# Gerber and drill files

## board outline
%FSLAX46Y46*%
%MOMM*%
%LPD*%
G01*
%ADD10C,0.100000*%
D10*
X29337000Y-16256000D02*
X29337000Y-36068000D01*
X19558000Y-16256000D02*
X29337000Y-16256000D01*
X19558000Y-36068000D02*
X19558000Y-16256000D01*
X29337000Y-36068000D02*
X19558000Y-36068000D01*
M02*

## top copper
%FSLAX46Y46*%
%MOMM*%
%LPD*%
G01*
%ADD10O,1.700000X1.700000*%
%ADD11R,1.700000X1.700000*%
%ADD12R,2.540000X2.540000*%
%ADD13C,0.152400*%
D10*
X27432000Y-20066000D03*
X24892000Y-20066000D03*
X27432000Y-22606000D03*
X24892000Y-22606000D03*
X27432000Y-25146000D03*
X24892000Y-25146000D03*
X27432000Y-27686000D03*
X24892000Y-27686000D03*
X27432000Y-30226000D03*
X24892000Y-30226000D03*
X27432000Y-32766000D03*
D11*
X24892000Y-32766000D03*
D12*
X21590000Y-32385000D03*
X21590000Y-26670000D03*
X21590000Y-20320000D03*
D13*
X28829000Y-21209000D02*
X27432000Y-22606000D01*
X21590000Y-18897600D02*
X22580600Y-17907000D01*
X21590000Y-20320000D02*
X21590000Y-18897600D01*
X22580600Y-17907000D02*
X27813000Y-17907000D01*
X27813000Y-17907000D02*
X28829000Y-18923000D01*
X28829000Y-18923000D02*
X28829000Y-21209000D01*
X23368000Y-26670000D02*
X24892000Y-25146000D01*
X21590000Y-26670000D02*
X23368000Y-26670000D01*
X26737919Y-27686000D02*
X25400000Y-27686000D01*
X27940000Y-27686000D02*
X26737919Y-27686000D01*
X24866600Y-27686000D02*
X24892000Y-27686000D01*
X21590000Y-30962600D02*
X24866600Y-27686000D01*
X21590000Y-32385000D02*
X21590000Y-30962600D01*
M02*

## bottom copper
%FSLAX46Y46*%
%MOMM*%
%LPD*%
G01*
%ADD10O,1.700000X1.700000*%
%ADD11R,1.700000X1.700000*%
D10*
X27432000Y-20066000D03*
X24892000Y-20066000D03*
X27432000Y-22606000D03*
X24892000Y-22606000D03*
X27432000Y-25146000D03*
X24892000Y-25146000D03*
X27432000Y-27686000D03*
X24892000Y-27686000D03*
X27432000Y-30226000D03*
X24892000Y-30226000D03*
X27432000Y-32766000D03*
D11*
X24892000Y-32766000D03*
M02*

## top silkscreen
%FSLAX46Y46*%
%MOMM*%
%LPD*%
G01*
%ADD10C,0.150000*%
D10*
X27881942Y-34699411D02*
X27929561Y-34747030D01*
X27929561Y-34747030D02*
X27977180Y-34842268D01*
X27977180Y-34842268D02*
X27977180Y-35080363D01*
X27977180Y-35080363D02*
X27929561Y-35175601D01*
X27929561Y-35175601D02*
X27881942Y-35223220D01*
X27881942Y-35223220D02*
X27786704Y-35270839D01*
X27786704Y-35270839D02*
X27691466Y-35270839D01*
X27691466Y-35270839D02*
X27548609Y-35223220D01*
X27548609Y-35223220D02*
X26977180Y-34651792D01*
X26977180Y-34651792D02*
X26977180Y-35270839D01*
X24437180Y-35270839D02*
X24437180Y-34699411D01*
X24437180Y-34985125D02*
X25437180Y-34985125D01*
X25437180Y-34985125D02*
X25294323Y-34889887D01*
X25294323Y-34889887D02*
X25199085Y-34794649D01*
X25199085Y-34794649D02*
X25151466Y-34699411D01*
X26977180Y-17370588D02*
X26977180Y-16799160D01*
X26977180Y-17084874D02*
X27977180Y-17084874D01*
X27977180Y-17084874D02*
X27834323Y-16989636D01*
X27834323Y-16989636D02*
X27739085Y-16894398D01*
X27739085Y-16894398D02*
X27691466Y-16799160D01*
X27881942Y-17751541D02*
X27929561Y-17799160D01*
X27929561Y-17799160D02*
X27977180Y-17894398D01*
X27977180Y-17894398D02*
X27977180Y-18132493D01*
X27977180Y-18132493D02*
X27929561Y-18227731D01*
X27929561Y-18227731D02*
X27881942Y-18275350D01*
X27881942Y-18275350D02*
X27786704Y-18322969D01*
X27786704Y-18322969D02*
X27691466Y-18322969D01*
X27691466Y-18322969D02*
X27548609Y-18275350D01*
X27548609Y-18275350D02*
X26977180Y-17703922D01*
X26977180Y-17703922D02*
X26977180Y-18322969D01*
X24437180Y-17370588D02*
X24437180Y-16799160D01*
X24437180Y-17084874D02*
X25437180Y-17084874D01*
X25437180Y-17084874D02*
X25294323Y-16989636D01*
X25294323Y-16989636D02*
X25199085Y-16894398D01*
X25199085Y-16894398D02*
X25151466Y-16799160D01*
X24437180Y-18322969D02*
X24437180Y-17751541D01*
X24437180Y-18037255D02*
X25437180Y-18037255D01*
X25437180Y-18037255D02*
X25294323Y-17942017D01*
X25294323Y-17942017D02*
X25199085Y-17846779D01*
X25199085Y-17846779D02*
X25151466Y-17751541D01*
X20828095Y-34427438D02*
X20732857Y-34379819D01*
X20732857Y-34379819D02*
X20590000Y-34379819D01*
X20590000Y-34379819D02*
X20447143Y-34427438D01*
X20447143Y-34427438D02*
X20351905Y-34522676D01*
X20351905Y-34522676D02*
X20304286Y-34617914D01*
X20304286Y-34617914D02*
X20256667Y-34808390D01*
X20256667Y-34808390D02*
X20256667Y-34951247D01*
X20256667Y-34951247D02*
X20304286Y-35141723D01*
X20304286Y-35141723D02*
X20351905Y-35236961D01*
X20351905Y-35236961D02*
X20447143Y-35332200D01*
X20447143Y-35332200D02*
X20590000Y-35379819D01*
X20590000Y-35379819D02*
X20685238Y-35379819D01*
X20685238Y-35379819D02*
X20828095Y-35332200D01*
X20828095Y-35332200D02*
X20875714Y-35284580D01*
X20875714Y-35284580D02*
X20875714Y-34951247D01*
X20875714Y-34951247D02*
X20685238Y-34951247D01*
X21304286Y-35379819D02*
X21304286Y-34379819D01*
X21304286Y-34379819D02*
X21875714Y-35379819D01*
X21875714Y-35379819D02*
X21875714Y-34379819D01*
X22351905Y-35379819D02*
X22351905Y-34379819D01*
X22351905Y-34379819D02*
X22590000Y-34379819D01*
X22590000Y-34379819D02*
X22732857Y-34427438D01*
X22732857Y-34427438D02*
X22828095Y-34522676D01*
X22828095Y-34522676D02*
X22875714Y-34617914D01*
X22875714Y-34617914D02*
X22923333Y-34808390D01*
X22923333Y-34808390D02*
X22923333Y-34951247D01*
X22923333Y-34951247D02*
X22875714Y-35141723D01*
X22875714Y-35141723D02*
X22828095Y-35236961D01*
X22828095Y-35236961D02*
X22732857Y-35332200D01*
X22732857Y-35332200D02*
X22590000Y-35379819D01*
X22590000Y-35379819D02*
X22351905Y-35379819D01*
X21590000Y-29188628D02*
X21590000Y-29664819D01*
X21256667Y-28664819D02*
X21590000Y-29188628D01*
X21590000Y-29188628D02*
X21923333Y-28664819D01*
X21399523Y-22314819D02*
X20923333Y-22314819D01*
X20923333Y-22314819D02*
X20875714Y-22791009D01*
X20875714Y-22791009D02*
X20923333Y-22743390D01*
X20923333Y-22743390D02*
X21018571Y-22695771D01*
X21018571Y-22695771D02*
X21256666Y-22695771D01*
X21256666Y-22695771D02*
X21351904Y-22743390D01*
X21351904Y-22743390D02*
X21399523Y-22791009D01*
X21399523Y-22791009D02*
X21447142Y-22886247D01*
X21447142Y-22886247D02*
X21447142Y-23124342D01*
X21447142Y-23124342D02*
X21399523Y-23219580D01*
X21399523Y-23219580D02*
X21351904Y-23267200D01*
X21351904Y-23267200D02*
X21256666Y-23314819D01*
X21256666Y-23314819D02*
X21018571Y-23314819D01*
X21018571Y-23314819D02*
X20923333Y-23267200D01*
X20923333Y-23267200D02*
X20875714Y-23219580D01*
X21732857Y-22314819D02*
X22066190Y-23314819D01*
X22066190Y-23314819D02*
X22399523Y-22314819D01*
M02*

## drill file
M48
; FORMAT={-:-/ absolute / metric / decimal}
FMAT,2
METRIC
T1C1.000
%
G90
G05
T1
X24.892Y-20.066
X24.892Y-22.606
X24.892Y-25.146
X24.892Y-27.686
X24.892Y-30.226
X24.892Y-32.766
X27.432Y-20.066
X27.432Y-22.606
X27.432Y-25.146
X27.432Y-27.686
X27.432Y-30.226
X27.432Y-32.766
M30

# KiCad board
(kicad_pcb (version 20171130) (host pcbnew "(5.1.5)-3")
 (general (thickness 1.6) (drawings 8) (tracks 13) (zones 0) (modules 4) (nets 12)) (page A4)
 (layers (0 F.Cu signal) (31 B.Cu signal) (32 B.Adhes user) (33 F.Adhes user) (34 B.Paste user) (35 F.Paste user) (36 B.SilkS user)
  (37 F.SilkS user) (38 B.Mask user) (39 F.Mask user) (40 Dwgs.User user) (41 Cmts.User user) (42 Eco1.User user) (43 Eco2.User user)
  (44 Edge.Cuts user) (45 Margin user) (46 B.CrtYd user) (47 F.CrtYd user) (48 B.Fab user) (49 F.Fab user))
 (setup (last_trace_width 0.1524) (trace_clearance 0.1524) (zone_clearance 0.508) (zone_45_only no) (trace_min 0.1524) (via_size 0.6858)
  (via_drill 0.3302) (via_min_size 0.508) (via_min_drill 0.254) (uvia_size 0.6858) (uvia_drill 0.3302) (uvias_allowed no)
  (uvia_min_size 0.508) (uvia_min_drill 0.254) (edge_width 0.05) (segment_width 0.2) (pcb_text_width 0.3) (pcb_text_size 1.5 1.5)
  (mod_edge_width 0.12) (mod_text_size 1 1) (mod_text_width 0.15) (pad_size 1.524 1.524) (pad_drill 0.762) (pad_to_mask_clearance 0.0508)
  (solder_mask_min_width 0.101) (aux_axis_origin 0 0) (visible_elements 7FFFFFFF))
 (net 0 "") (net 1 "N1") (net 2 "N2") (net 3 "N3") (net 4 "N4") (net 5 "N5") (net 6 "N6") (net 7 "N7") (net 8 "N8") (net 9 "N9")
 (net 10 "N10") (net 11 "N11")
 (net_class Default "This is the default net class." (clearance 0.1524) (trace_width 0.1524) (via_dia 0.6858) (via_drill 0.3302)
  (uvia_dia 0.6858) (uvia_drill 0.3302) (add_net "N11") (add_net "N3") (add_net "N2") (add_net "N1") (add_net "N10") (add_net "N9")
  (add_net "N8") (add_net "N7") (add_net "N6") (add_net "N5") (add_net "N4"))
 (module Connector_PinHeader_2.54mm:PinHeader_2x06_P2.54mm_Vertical (layer B.Cu) (at 24.892 32.766)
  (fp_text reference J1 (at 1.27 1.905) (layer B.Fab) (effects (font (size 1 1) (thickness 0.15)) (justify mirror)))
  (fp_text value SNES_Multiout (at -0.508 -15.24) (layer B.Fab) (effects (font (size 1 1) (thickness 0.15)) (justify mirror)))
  (pad 12 thru_hole oval (at 2.54 -12.7) (size 1.7 1.7) (drill 1) (layers *.Cu *.Mask) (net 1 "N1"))
  (pad 11 thru_hole oval (at 0 -12.7) (size 1.7 1.7) (drill 1) (layers *.Cu *.Mask) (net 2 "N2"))
  (pad 10 thru_hole oval (at 2.54 -10.16) (size 1.7 1.7) (drill 1) (layers *.Cu *.Mask) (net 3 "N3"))
  (pad 9 thru_hole oval (at 0 -10.16) (size 1.7 1.7) (drill 1) (layers *.Cu *.Mask) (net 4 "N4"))
  (pad 8 thru_hole oval (at 2.54 -7.62) (size 1.7 1.7) (drill 1) (layers *.Cu *.Mask) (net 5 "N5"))
  (pad 7 thru_hole oval (at 0 -7.62) (size 1.7 1.7) (drill 1) (layers *.Cu *.Mask) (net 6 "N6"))
  (pad 6 thru_hole oval (at 2.54 -5.08) (size 1.7 1.7) (drill 1) (layers *.Cu *.Mask) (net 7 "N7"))
  (pad 5 thru_hole oval (at 0 -5.08) (size 1.7 1.7) (drill 1) (layers *.Cu *.Mask) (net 7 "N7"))
  (pad 4 thru_hole oval (at 2.54 -2.54) (size 1.7 1.7) (drill 1) (layers *.Cu *.Mask) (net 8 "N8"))
  (pad 3 thru_hole oval (at 0 -2.54) (size 1.7 1.7) (drill 1) (layers *.Cu *.Mask) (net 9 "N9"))
  (pad 2 thru_hole oval (at 2.54 0) (size 1.7 1.7) (drill 1) (layers *.Cu *.Mask) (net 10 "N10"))
  (pad 1 thru_hole rect (at 0 0) (size 1.7 1.7) (drill 1) (layers *.Cu *.Mask) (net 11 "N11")))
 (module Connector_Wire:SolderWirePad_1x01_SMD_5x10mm (layer F.Cu) (at 21.59 32.385)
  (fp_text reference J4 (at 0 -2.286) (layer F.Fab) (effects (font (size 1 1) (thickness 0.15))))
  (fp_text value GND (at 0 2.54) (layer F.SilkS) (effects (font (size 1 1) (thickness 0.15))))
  (pad 1 smd rect (at 0 0) (size 2.54 2.54) (layers F.Cu F.Paste F.Mask) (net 7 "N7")))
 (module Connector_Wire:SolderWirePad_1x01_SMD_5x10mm (layer F.Cu) (at 21.59 26.67)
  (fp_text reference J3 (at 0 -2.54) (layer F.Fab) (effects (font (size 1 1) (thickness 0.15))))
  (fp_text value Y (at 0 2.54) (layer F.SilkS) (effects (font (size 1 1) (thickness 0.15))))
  (pad 1 smd rect (at 0 0) (size 2.54 2.54) (layers F.Cu F.Paste F.Mask) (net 6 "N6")))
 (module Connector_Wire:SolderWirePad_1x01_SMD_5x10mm (layer F.Cu) (at 21.59 20.32)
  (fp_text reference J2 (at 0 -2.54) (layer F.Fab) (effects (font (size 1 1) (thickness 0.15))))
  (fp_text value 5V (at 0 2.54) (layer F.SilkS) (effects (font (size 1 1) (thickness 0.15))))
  (pad 1 smd rect (at 0 0) (size 2.54 2.54) (layers F.Cu F.Paste F.Mask) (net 3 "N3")))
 (gr_line (start 29.337 16.256) (end 29.337 36.068) (layer Edge.Cuts) (width 0.1))
 (gr_line (start 19.558 16.256) (end 29.337 16.256) (layer Edge.Cuts) (width 0.1))
 (gr_line (start 19.558 36.068) (end 19.558 16.256) (layer Edge.Cuts) (width 0.1))
 (gr_line (start 29.337 36.068) (end 19.558 36.068) (layer Edge.Cuts) (width 0.1))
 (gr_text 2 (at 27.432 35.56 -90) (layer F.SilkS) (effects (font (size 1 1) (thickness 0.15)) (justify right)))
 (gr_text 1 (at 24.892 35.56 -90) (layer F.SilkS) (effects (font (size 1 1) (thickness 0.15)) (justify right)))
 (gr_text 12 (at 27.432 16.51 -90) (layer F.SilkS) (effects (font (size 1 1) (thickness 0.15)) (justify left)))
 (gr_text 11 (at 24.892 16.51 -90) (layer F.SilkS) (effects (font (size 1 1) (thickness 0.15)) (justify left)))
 (segment (start 28.829 21.209) (end 27.432 22.606) (width 0.1524) (layer F.Cu) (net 3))
 (segment (start 21.59 18.8976) (end 22.5806 17.907) (width 0.1524) (layer F.Cu) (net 3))
 (segment (start 21.59 20.32) (end 21.59 18.8976) (width 0.1524) (layer F.Cu) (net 3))
 (segment (start 22.5806 17.907) (end 27.813 17.907) (width 0.1524) (layer F.Cu) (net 3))
 (segment (start 27.813 17.907) (end 28.829 18.923) (width 0.1524) (layer F.Cu) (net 3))
 (segment (start 28.829 18.923) (end 28.829 21.209) (width 0.1524) (layer F.Cu) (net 3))
 (segment (start 23.368 26.67) (end 24.892 25.146) (width 0.1524) (layer F.Cu) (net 6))
 (segment (start 21.59 26.67) (end 23.368 26.67) (width 0.1524) (layer F.Cu) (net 6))
 (segment (start 26.737919 27.686) (end 25.4 27.686) (width 0.1524) (layer F.Cu) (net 7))
 (segment (start 27.94 27.686) (end 26.737919 27.686) (width 0.1524) (layer F.Cu) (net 7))
 (segment (start 24.8666 27.686) (end 24.892 27.686) (width 0.1524) (layer F.Cu) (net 7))
 (segment (start 21.59 30.9626) (end 24.8666 27.686) (width 0.1524) (layer F.Cu) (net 7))
 (segment (start 21.59 32.385) (end 21.59 30.9626) (width 0.1524) (layer F.Cu) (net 7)))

